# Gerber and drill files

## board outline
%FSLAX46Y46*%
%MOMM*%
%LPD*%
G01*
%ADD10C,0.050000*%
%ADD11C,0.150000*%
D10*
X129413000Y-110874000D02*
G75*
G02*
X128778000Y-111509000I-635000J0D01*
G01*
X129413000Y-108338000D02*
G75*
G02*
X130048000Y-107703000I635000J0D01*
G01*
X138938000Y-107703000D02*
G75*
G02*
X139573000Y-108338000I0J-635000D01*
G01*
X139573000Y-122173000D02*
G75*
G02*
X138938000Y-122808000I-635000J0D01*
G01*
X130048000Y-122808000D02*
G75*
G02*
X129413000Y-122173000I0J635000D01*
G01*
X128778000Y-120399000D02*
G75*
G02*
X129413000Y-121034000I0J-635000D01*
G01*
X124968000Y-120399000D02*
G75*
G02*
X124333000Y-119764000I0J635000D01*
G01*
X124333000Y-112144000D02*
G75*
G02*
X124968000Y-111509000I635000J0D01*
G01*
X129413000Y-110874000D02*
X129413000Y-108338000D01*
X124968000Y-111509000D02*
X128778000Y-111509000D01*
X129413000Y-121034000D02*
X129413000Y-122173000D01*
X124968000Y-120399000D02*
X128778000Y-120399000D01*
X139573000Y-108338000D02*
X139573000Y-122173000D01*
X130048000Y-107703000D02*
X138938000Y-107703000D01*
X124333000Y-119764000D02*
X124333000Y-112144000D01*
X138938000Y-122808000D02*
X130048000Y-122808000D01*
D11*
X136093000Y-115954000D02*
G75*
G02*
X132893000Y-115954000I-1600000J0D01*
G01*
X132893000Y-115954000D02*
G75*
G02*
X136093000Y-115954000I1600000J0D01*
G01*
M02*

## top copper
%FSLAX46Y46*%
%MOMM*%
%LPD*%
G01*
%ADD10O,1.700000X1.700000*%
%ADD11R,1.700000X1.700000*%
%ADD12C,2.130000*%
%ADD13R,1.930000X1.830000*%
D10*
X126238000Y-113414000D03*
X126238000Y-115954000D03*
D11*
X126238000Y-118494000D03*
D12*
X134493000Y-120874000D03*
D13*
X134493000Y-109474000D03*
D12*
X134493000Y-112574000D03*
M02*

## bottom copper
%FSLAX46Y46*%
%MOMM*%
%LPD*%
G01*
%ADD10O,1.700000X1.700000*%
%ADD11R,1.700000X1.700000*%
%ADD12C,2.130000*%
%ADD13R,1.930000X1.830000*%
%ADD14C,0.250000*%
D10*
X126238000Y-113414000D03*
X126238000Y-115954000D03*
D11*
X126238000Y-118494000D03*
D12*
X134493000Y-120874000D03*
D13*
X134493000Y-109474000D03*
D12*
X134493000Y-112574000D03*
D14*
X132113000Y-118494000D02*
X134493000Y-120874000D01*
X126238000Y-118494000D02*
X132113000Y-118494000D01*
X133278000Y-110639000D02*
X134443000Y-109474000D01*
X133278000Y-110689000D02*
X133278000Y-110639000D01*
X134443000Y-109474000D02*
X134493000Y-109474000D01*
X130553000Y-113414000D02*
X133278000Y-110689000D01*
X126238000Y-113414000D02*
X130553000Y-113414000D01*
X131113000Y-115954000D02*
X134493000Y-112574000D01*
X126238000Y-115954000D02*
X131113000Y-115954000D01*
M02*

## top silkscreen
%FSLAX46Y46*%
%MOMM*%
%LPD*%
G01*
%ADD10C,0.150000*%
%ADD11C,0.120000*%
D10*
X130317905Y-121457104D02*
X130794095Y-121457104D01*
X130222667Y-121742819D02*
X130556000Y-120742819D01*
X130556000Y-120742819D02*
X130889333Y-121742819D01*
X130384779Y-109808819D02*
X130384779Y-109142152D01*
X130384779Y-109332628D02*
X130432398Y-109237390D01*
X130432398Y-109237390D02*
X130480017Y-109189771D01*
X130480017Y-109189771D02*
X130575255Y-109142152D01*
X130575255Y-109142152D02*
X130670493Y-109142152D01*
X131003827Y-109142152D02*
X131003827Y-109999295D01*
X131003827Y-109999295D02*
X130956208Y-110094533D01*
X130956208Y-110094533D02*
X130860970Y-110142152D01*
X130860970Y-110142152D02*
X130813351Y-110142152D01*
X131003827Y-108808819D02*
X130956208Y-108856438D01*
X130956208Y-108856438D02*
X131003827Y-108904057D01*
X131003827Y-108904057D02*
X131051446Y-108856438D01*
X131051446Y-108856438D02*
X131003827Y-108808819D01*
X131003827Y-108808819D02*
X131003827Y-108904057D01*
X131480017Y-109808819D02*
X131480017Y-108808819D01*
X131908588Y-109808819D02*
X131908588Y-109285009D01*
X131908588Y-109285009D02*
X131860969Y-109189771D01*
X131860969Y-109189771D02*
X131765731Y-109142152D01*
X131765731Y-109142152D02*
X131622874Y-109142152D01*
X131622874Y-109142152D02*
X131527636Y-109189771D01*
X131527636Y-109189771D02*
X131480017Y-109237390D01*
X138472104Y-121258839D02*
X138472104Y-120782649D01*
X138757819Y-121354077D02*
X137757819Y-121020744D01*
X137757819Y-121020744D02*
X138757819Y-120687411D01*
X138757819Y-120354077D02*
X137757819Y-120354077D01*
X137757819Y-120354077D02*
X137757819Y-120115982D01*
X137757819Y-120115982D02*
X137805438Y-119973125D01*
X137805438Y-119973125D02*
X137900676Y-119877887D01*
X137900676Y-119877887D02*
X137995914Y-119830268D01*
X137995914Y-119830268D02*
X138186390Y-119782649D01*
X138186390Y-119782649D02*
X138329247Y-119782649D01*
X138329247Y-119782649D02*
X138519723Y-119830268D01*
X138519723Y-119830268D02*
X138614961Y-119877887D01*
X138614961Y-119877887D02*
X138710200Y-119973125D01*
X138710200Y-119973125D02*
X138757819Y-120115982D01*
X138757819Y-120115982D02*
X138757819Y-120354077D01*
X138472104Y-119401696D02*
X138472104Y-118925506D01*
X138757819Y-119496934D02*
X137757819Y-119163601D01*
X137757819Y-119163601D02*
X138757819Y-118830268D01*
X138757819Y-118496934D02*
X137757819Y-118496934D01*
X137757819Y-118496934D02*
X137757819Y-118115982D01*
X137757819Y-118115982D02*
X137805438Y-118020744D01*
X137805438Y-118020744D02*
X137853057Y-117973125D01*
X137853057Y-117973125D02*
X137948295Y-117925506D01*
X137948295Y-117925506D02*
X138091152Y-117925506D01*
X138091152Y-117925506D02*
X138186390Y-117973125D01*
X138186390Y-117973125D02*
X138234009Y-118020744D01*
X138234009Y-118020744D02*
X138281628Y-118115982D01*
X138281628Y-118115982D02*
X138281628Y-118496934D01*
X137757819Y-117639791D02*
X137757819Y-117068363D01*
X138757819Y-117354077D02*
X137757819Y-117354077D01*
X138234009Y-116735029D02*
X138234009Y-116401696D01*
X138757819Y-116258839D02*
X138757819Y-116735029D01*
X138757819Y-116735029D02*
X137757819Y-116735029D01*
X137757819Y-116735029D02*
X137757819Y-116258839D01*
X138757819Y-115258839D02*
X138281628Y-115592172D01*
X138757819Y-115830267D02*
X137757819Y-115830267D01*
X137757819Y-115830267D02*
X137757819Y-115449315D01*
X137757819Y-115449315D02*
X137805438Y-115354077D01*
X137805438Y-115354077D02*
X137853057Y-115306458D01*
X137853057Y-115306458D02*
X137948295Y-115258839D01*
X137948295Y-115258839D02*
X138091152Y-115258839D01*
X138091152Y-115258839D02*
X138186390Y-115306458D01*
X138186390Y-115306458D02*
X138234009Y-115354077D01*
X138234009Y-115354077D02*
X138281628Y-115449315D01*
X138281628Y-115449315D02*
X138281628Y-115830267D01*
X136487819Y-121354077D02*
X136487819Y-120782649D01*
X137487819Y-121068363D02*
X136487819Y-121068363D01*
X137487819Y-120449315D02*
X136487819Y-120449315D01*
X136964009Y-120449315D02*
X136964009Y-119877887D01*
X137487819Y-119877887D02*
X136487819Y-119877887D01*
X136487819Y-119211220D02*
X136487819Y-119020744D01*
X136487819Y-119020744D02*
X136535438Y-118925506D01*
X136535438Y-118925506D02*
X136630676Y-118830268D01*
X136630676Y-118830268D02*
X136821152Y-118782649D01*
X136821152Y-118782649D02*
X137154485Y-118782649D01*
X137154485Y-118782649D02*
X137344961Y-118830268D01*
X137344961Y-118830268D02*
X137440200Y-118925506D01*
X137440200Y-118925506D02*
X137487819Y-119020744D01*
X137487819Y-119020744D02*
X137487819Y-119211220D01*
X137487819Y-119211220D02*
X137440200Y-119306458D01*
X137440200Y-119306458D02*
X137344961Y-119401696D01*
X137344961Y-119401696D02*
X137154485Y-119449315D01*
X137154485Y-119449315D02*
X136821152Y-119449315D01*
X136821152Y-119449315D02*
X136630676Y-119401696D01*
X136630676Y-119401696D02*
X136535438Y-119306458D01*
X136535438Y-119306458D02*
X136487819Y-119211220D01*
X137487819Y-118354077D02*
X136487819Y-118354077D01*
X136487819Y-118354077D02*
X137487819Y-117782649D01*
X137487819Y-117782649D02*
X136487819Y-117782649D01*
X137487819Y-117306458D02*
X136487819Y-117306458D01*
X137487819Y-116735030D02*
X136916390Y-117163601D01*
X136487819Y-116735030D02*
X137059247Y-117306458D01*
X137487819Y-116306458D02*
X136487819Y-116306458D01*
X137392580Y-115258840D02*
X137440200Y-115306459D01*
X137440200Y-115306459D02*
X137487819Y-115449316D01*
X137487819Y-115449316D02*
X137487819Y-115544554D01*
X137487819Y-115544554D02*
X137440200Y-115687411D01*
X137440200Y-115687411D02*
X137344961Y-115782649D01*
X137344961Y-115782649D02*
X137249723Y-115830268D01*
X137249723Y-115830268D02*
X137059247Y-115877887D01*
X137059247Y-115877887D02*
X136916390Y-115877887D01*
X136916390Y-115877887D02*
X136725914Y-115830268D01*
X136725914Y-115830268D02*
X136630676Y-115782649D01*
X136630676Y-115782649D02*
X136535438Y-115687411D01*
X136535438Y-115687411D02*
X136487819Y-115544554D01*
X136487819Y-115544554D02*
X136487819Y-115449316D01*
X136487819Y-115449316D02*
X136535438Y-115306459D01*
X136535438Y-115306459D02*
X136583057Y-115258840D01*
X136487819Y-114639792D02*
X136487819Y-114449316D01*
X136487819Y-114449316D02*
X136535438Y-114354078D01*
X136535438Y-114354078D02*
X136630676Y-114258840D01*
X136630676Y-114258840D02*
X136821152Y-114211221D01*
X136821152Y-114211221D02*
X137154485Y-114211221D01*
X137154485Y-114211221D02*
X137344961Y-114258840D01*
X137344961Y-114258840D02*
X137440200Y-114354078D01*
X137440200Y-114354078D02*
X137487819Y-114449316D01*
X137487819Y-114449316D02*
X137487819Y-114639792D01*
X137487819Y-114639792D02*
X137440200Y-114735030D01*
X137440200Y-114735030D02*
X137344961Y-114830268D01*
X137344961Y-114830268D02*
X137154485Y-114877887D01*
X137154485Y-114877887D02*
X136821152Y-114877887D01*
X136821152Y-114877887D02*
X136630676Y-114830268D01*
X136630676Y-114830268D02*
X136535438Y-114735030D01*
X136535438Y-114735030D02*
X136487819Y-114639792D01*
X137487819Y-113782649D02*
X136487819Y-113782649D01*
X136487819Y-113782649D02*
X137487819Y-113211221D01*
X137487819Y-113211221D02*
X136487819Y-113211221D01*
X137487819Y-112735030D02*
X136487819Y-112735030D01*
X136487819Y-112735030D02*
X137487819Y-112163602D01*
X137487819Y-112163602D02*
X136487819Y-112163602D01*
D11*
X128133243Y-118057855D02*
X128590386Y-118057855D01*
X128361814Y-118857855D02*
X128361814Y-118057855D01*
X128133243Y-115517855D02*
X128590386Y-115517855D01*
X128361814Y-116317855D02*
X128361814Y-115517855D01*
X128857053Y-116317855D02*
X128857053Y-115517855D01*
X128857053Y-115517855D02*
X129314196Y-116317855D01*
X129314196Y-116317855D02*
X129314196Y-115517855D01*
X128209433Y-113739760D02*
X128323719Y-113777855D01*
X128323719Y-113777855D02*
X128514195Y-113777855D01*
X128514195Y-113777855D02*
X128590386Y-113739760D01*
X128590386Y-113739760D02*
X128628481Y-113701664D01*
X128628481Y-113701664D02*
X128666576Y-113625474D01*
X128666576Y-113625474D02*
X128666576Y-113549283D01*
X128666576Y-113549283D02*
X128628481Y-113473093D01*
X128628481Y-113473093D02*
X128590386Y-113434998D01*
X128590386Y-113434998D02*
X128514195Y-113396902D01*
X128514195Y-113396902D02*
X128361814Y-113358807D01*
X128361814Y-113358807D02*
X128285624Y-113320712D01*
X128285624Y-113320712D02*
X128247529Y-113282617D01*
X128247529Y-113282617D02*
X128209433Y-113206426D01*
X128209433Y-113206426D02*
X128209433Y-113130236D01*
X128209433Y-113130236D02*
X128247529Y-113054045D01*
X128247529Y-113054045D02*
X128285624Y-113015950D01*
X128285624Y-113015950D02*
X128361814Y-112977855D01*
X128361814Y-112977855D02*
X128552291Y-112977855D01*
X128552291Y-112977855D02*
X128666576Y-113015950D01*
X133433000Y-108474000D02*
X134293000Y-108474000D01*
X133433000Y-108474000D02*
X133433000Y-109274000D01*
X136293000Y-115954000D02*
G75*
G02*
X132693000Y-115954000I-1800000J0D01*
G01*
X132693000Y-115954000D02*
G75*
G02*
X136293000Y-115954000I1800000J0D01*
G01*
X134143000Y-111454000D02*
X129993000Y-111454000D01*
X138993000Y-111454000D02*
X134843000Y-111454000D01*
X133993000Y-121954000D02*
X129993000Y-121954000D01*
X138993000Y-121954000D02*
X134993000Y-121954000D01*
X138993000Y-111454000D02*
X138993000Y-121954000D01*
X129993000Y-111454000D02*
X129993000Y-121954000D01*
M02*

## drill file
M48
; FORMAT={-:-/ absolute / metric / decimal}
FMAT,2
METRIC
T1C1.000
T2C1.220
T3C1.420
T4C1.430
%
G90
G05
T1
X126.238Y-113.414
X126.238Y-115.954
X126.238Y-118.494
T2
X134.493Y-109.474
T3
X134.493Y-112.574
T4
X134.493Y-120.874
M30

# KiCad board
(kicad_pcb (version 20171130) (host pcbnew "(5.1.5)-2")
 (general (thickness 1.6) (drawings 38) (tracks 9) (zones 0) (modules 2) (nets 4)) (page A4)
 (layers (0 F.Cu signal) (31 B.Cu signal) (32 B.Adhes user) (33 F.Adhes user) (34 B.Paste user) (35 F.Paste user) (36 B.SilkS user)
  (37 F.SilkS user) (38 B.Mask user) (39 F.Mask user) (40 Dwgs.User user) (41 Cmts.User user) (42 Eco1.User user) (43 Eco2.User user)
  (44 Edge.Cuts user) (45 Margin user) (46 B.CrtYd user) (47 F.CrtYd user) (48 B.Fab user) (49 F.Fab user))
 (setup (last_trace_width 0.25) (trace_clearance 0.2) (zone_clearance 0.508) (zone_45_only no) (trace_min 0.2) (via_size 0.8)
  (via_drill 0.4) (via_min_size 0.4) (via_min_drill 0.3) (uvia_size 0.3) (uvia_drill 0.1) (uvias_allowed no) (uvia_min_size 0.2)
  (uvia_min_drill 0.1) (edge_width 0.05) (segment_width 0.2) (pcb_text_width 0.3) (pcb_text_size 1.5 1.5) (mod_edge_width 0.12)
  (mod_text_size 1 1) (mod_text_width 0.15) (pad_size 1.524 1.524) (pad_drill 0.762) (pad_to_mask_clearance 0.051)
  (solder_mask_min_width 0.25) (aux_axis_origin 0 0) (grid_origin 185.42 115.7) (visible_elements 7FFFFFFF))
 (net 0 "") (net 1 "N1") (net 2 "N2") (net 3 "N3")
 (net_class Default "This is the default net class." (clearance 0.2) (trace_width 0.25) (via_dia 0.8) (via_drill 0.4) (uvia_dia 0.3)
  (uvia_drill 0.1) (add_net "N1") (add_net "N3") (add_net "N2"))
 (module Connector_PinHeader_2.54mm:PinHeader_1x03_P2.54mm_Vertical (layer B.Cu) (at 126.238 118.494)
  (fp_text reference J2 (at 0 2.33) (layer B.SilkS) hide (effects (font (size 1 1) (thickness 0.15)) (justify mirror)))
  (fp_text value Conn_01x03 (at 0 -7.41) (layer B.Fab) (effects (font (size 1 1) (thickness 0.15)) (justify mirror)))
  (pad 3 thru_hole oval (at 0 -5.08) (size 1.7 1.7) (drill 1) (layers *.Cu *.Mask) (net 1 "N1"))
  (pad 2 thru_hole oval (at 0 -2.54) (size 1.7 1.7) (drill 1) (layers *.Cu *.Mask) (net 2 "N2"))
  (pad 1 thru_hole rect (at 0 0) (size 1.7 1.7) (drill 1) (layers *.Cu *.Mask) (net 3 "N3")))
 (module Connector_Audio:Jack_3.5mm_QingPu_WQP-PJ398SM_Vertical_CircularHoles (layer F.Cu) (at 134.493 109.474)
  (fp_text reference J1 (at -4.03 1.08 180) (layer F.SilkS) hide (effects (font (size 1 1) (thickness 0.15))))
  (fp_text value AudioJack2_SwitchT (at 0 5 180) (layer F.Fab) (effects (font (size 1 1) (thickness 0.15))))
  (fp_line (start -1.06 -1) (end -0.2 -1) (layer F.SilkS) (width 0.12))
  (fp_line (start -1.06 -1) (end -1.06 -0.2) (layer F.SilkS) (width 0.12))
  (fp_circle (center 0 6.48) (end 1.8 6.48) (layer F.SilkS) (width 0.12))
  (fp_line (start -0.35 1.98) (end -4.5 1.98) (layer F.SilkS) (width 0.12))
  (fp_line (start 4.5 1.98) (end 0.35 1.98) (layer F.SilkS) (width 0.12))
  (fp_line (start -0.5 12.48) (end -4.5 12.48) (layer F.SilkS) (width 0.12))
  (fp_line (start 4.5 12.48) (end 0.5 12.48) (layer F.SilkS) (width 0.12))
  (fp_line (start 4.5 1.98) (end 4.5 12.48) (layer F.SilkS) (width 0.12))
  (fp_line (start -4.5 1.98) (end -4.5 12.48) (layer F.SilkS) (width 0.12))
  (pad T thru_hole circle (at 0 11.4 180) (size 2.13 2.13) (drill 1.43) (layers *.Cu *.Mask) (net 3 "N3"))
  (pad S thru_hole rect (at 0 0 180) (size 1.93 1.83) (drill 1.22) (layers *.Cu *.Mask) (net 1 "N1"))
  (pad TN thru_hole circle (at 0 3.1 180) (size 2.13 2.13) (drill 1.42) (layers *.Cu *.Mask) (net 2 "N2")))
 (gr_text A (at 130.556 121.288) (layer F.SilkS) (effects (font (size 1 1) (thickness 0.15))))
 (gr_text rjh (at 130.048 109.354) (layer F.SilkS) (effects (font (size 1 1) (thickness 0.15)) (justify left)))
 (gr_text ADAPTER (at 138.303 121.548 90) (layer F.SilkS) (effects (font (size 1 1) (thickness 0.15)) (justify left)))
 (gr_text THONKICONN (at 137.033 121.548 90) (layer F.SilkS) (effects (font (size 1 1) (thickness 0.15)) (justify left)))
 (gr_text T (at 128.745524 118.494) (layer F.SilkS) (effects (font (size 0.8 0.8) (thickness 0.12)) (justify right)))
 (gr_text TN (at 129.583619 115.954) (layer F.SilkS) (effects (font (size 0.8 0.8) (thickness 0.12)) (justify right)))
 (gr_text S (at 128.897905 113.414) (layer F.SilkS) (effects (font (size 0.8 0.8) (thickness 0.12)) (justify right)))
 (gr_arc (start 128.778 110.874) (end 128.778 111.509) (angle -90) (layer Edge.Cuts) (width 0.05))
 (gr_arc (start 130.048 108.338) (end 130.048 107.703) (angle -90) (layer Edge.Cuts) (width 0.05))
 (gr_arc (start 138.938 108.338) (end 139.573 108.338) (angle -90) (layer Edge.Cuts) (width 0.05))
 (gr_arc (start 138.938 122.173) (end 138.938 122.808) (angle -90) (layer Edge.Cuts) (width 0.05))
 (gr_arc (start 130.048 122.173) (end 129.413 122.173) (angle -90) (layer Edge.Cuts) (width 0.05))
 (gr_arc (start 128.778 121.034) (end 129.413 121.034) (angle -90) (layer Edge.Cuts) (width 0.05))
 (gr_arc (start 124.968 119.764) (end 124.333 119.764) (angle -90) (layer Edge.Cuts) (width 0.05))
 (gr_arc (start 124.968 112.144) (end 124.968 111.509) (angle -90) (layer Edge.Cuts) (width 0.05))
 (gr_line (start 129.413 110.874) (end 129.413 108.338) (layer Edge.Cuts) (width 0.05))
 (gr_line (start 124.968 111.509) (end 128.778 111.509) (layer Edge.Cuts) (width 0.05))
 (gr_line (start 129.413 121.034) (end 129.413 122.173) (layer Edge.Cuts) (width 0.05))
 (gr_line (start 124.968 120.399) (end 128.778 120.399) (layer Edge.Cuts) (width 0.05))
 (gr_line (start 139.573 108.338) (end 139.573 122.173) (layer Edge.Cuts) (width 0.05))
 (gr_line (start 130.048 107.703) (end 138.938 107.703) (layer Edge.Cuts) (width 0.05))
 (gr_line (start 124.333 119.764) (end 124.333 112.144) (layer Edge.Cuts) (width 0.05))
 (gr_line (start 138.938 122.808) (end 130.048 122.808) (layer Edge.Cuts) (width 0.05))
 (gr_circle (center 134.493 115.954) (end 136.093 115.954) (layer Edge.Cuts) (width 0.15))
 (segment (start 132.113 118.494) (end 134.493 120.874) (width 0.25) (layer B.Cu) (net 3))
 (segment (start 126.238 118.494) (end 132.113 118.494) (width 0.25) (layer B.Cu) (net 3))
 (segment (start 133.278 110.639) (end 134.443 109.474) (width 0.25) (layer B.Cu) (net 1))
 (segment (start 133.278 110.689) (end 133.278 110.639) (width 0.25) (layer B.Cu) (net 1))
 (segment (start 134.443 109.474) (end 134.493 109.474) (width 0.25) (layer B.Cu) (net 1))
 (segment (start 130.553 113.414) (end 133.278 110.689) (width 0.25) (layer B.Cu) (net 1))
 (segment (start 126.238 113.414) (end 130.553 113.414) (width 0.25) (layer B.Cu) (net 1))
 (segment (start 131.113 115.954) (end 134.493 112.574) (width 0.25) (layer B.Cu) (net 2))
 (segment (start 126.238 115.954) (end 131.113 115.954) (width 0.25) (layer B.Cu) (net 2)))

